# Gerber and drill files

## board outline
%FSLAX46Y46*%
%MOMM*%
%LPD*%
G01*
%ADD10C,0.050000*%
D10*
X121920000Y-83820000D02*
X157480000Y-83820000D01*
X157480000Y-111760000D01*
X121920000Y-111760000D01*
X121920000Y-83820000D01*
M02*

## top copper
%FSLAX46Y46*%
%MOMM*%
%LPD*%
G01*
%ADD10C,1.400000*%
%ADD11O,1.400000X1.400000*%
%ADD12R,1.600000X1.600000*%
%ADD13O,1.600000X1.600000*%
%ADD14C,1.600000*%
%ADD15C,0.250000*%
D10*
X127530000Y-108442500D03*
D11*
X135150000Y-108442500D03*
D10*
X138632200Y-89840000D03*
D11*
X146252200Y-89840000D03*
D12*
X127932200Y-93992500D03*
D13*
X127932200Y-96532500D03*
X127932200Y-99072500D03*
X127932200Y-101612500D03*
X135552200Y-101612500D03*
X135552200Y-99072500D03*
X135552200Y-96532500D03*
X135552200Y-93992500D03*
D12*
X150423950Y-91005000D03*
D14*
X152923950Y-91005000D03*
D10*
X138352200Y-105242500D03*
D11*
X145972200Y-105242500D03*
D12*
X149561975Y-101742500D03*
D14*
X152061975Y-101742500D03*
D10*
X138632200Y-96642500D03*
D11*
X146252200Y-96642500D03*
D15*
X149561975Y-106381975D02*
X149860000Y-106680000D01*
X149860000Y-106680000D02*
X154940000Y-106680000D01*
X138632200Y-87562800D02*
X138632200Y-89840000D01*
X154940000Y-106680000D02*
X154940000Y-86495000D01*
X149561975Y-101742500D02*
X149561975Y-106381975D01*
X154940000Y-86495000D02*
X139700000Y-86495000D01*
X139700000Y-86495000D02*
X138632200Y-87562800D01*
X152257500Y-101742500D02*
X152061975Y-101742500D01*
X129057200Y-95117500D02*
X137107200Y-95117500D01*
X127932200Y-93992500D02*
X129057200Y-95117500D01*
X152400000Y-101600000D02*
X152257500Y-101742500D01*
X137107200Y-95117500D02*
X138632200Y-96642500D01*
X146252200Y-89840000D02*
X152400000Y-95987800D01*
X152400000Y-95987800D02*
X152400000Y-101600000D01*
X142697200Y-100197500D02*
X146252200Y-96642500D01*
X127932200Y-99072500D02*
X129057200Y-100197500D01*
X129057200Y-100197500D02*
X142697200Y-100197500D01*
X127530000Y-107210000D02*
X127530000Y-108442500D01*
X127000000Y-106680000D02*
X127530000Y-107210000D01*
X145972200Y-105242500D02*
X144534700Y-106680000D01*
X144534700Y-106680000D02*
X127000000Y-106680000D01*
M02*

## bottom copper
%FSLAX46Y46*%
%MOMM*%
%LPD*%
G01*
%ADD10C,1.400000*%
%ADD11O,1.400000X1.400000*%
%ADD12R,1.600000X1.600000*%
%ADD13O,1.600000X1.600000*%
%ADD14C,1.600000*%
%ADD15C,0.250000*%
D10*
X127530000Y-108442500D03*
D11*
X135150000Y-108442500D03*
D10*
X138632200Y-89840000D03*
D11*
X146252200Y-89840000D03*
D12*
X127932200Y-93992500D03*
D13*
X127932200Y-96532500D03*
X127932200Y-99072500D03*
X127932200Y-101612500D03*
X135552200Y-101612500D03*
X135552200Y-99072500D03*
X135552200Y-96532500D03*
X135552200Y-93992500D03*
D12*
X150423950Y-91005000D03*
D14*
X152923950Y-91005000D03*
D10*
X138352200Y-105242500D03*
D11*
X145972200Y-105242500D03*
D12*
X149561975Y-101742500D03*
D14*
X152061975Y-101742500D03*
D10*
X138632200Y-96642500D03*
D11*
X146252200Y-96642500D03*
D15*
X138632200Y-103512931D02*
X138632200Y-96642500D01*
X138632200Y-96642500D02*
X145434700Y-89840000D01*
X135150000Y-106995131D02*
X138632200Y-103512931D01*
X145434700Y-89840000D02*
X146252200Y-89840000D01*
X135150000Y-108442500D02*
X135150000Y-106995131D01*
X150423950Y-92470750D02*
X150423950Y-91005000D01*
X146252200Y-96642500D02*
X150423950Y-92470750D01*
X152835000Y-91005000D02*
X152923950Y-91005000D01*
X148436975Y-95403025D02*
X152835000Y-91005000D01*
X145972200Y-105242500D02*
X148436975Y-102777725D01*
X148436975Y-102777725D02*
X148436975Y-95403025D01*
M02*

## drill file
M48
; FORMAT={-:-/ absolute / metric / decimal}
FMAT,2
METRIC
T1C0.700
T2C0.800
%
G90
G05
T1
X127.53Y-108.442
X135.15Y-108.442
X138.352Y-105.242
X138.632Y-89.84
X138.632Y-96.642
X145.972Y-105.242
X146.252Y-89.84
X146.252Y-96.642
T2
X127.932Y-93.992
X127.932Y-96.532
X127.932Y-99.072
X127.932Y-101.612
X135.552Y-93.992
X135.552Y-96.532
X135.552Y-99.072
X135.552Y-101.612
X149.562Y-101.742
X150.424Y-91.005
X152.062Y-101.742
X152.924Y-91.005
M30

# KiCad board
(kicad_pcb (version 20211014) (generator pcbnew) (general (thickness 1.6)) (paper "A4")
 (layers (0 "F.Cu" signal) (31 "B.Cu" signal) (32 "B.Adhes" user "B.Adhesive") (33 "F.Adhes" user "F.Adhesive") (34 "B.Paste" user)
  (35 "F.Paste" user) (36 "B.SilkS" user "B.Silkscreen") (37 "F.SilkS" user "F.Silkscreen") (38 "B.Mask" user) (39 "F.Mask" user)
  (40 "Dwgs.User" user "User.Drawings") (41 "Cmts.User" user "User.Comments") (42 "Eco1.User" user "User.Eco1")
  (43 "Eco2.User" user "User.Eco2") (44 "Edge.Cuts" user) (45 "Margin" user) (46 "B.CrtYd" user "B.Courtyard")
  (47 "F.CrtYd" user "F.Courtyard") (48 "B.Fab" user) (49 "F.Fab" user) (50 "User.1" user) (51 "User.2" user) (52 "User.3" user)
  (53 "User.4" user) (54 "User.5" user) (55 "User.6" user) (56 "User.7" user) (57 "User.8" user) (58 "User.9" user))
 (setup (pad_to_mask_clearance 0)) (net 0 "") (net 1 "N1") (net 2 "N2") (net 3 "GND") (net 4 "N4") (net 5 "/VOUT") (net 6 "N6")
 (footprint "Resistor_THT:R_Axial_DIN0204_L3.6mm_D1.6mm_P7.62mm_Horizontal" (layer "F.Cu") (at 127.53 108.4425)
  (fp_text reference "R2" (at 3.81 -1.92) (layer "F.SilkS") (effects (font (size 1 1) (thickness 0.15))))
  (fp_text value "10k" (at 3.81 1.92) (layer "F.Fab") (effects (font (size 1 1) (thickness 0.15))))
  (pad "1" thru_hole circle (at 0 0) (size 1.4 1.4) (drill 0.7) (layers *.Cu *.Mask) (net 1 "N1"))
  (pad "2" thru_hole oval (at 7.62 0) (size 1.4 1.4) (drill 0.7) (layers *.Cu *.Mask) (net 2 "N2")))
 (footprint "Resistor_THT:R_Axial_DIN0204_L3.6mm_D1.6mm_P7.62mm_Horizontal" (layer "F.Cu") (at 138.6322 89.84)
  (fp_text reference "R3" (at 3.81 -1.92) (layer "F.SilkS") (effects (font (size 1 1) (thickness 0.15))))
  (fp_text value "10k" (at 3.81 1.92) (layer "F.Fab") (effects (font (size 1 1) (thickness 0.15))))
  (pad "1" thru_hole circle (at 0 0) (size 1.4 1.4) (drill 0.7) (layers *.Cu *.Mask) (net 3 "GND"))
  (pad "2" thru_hole oval (at 7.62 0) (size 1.4 1.4) (drill 0.7) (layers *.Cu *.Mask) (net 2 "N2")))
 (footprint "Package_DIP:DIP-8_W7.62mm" (layer "F.Cu") (at 127.9322 93.9925)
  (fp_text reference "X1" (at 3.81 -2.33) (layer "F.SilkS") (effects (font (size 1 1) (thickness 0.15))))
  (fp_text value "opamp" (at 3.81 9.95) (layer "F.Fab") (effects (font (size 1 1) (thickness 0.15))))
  (pad "1" thru_hole rect (at 0 0) (size 1.6 1.6) (drill 0.8) (layers *.Cu *.Mask) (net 2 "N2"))
  (pad "2" thru_hole oval (at 0 2.54) (size 1.6 1.6) (drill 0.8) (layers *.Cu *.Mask) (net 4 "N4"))
  (pad "3" thru_hole oval (at 0 5.08) (size 1.6 1.6) (drill 0.8) (layers *.Cu *.Mask) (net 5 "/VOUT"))
  (pad "4" thru_hole oval (at 0 7.62) (size 1.6 1.6) (drill 0.8) (layers *.Cu *.Mask))
  (pad "5" thru_hole oval (at 7.62 7.62) (size 1.6 1.6) (drill 0.8) (layers *.Cu *.Mask))
  (pad "6" thru_hole oval (at 7.62 5.08) (size 1.6 1.6) (drill 0.8) (layers *.Cu *.Mask))
  (pad "7" thru_hole oval (at 7.62 2.54) (size 1.6 1.6) (drill 0.8) (layers *.Cu *.Mask))
  (pad "8" thru_hole oval (at 7.62 0) (size 1.6 1.6) (drill 0.8) (layers *.Cu *.Mask)))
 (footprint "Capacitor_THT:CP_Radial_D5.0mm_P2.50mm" (layer "F.Cu") (at 150.42395 91.005)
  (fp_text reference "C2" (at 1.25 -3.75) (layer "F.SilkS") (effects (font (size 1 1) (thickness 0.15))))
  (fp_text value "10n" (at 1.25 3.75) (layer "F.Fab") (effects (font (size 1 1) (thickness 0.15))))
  (pad "1" thru_hole rect (at 0 0) (size 1.6 1.6) (drill 0.8) (layers *.Cu *.Mask) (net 5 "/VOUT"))
  (pad "2" thru_hole circle (at 2.5 0) (size 1.6 1.6) (drill 0.8) (layers *.Cu *.Mask) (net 1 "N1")))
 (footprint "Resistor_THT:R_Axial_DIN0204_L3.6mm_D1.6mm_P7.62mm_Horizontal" (layer "F.Cu") (at 138.3522 105.2425)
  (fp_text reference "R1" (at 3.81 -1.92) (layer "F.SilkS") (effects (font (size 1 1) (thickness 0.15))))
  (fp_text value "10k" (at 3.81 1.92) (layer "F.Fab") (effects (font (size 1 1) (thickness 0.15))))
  (pad "1" thru_hole circle (at 0 0) (size 1.4 1.4) (drill 0.7) (layers *.Cu *.Mask) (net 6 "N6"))
  (pad "2" thru_hole oval (at 7.62 0) (size 1.4 1.4) (drill 0.7) (layers *.Cu *.Mask) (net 1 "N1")))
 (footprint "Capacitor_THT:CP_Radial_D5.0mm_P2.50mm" (layer "F.Cu") (at 149.561975 101.7425)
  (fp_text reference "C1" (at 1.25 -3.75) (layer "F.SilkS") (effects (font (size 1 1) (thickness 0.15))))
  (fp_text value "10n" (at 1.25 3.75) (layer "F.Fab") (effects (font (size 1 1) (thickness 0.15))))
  (pad "1" thru_hole rect (at 0 0) (size 1.6 1.6) (drill 0.8) (layers *.Cu *.Mask) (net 3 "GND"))
  (pad "2" thru_hole circle (at 2.5 0) (size 1.6 1.6) (drill 0.8) (layers *.Cu *.Mask) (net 2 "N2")))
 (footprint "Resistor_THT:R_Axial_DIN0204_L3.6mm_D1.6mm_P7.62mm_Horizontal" (layer "F.Cu") (at 138.6322 96.6425)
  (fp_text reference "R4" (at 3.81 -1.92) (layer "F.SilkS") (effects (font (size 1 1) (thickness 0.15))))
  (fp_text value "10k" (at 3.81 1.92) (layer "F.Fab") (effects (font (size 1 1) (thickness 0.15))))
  (pad "1" thru_hole circle (at 0 0) (size 1.4 1.4) (drill 0.7) (layers *.Cu *.Mask) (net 2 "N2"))
  (pad "2" thru_hole oval (at 7.62 0) (size 1.4 1.4) (drill 0.7) (layers *.Cu *.Mask) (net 5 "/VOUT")))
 (gr_rect (start 121.92 83.82) (end 157.48 111.76) (layer "Edge.Cuts") (width 0.05) (fill none))
 (segment (start 149.561975 106.381975) (end 149.86 106.68) (width 0.25) (layer "F.Cu") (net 3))
 (segment (start 149.86 106.68) (end 154.94 106.68) (width 0.25) (layer "F.Cu") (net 3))
 (segment (start 138.6322 87.5628) (end 138.6322 89.84) (width 0.25) (layer "F.Cu") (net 3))
 (segment (start 154.94 106.68) (end 154.94 86.495) (width 0.25) (layer "F.Cu") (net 3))
 (segment (start 149.561975 101.7425) (end 149.561975 106.381975) (width 0.25) (layer "F.Cu") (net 3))
 (segment (start 154.94 86.495) (end 139.7 86.495) (width 0.25) (layer "F.Cu") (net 3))
 (segment (start 139.7 86.495) (end 138.6322 87.5628) (width 0.25) (layer "F.Cu") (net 3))
 (segment (start 152.2575 101.7425) (end 152.061975 101.7425) (width 0.25) (layer "F.Cu") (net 2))
 (segment (start 129.0572 95.1175) (end 137.1072 95.1175) (width 0.25) (layer "F.Cu") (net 2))
 (segment (start 127.9322 93.9925) (end 129.0572 95.1175) (width 0.25) (layer "F.Cu") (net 2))
 (segment (start 152.4 101.6) (end 152.2575 101.7425) (width 0.25) (layer "F.Cu") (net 2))
 (segment (start 137.1072 95.1175) (end 138.6322 96.6425) (width 0.25) (layer "F.Cu") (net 2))
 (segment (start 146.2522 89.84) (end 152.4 95.9878) (width 0.25) (layer "F.Cu") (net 2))
 (segment (start 152.4 95.9878) (end 152.4 101.6) (width 0.25) (layer "F.Cu") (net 2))
 (segment (start 138.6322 103.512931) (end 138.6322 96.6425) (width 0.25) (layer "B.Cu") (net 2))
 (segment (start 138.6322 96.6425) (end 145.4347 89.84) (width 0.25) (layer "B.Cu") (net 2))
 (segment (start 135.15 106.995131) (end 138.6322 103.512931) (width 0.25) (layer "B.Cu") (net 2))
 (segment (start 145.4347 89.84) (end 146.2522 89.84) (width 0.25) (layer "B.Cu") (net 2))
 (segment (start 135.15 108.4425) (end 135.15 106.995131) (width 0.25) (layer "B.Cu") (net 2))
 (segment (start 142.6972 100.1975) (end 146.2522 96.6425) (width 0.25) (layer "F.Cu") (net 5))
 (segment (start 127.9322 99.0725) (end 129.0572 100.1975) (width 0.25) (layer "F.Cu") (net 5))
 (segment (start 129.0572 100.1975) (end 142.6972 100.1975) (width 0.25) (layer "F.Cu") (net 5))
 (segment (start 150.42395 92.47075) (end 150.42395 91.005) (width 0.25) (layer "B.Cu") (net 5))
 (segment (start 146.2522 96.6425) (end 150.42395 92.47075) (width 0.25) (layer "B.Cu") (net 5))
 (segment (start 127.53 107.21) (end 127.53 108.4425) (width 0.25) (layer "F.Cu") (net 1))
 (segment (start 127 106.68) (end 127.53 107.21) (width 0.25) (layer "F.Cu") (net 1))
 (segment (start 145.9722 105.2425) (end 144.5347 106.68) (width 0.25) (layer "F.Cu") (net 1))
 (segment (start 144.5347 106.68) (end 127 106.68) (width 0.25) (layer "F.Cu") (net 1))
 (segment (start 152.835 91.005) (end 152.92395 91.005) (width 0.25) (layer "B.Cu") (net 1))
 (segment (start 148.436975 95.403025) (end 152.835 91.005) (width 0.25) (layer "B.Cu") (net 1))
 (segment (start 145.9722 105.2425) (end 148.436975 102.777725) (width 0.25) (layer "B.Cu") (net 1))
 (segment (start 148.436975 102.777725) (end 148.436975 95.403025) (width 0.25) (layer "B.Cu") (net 1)))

